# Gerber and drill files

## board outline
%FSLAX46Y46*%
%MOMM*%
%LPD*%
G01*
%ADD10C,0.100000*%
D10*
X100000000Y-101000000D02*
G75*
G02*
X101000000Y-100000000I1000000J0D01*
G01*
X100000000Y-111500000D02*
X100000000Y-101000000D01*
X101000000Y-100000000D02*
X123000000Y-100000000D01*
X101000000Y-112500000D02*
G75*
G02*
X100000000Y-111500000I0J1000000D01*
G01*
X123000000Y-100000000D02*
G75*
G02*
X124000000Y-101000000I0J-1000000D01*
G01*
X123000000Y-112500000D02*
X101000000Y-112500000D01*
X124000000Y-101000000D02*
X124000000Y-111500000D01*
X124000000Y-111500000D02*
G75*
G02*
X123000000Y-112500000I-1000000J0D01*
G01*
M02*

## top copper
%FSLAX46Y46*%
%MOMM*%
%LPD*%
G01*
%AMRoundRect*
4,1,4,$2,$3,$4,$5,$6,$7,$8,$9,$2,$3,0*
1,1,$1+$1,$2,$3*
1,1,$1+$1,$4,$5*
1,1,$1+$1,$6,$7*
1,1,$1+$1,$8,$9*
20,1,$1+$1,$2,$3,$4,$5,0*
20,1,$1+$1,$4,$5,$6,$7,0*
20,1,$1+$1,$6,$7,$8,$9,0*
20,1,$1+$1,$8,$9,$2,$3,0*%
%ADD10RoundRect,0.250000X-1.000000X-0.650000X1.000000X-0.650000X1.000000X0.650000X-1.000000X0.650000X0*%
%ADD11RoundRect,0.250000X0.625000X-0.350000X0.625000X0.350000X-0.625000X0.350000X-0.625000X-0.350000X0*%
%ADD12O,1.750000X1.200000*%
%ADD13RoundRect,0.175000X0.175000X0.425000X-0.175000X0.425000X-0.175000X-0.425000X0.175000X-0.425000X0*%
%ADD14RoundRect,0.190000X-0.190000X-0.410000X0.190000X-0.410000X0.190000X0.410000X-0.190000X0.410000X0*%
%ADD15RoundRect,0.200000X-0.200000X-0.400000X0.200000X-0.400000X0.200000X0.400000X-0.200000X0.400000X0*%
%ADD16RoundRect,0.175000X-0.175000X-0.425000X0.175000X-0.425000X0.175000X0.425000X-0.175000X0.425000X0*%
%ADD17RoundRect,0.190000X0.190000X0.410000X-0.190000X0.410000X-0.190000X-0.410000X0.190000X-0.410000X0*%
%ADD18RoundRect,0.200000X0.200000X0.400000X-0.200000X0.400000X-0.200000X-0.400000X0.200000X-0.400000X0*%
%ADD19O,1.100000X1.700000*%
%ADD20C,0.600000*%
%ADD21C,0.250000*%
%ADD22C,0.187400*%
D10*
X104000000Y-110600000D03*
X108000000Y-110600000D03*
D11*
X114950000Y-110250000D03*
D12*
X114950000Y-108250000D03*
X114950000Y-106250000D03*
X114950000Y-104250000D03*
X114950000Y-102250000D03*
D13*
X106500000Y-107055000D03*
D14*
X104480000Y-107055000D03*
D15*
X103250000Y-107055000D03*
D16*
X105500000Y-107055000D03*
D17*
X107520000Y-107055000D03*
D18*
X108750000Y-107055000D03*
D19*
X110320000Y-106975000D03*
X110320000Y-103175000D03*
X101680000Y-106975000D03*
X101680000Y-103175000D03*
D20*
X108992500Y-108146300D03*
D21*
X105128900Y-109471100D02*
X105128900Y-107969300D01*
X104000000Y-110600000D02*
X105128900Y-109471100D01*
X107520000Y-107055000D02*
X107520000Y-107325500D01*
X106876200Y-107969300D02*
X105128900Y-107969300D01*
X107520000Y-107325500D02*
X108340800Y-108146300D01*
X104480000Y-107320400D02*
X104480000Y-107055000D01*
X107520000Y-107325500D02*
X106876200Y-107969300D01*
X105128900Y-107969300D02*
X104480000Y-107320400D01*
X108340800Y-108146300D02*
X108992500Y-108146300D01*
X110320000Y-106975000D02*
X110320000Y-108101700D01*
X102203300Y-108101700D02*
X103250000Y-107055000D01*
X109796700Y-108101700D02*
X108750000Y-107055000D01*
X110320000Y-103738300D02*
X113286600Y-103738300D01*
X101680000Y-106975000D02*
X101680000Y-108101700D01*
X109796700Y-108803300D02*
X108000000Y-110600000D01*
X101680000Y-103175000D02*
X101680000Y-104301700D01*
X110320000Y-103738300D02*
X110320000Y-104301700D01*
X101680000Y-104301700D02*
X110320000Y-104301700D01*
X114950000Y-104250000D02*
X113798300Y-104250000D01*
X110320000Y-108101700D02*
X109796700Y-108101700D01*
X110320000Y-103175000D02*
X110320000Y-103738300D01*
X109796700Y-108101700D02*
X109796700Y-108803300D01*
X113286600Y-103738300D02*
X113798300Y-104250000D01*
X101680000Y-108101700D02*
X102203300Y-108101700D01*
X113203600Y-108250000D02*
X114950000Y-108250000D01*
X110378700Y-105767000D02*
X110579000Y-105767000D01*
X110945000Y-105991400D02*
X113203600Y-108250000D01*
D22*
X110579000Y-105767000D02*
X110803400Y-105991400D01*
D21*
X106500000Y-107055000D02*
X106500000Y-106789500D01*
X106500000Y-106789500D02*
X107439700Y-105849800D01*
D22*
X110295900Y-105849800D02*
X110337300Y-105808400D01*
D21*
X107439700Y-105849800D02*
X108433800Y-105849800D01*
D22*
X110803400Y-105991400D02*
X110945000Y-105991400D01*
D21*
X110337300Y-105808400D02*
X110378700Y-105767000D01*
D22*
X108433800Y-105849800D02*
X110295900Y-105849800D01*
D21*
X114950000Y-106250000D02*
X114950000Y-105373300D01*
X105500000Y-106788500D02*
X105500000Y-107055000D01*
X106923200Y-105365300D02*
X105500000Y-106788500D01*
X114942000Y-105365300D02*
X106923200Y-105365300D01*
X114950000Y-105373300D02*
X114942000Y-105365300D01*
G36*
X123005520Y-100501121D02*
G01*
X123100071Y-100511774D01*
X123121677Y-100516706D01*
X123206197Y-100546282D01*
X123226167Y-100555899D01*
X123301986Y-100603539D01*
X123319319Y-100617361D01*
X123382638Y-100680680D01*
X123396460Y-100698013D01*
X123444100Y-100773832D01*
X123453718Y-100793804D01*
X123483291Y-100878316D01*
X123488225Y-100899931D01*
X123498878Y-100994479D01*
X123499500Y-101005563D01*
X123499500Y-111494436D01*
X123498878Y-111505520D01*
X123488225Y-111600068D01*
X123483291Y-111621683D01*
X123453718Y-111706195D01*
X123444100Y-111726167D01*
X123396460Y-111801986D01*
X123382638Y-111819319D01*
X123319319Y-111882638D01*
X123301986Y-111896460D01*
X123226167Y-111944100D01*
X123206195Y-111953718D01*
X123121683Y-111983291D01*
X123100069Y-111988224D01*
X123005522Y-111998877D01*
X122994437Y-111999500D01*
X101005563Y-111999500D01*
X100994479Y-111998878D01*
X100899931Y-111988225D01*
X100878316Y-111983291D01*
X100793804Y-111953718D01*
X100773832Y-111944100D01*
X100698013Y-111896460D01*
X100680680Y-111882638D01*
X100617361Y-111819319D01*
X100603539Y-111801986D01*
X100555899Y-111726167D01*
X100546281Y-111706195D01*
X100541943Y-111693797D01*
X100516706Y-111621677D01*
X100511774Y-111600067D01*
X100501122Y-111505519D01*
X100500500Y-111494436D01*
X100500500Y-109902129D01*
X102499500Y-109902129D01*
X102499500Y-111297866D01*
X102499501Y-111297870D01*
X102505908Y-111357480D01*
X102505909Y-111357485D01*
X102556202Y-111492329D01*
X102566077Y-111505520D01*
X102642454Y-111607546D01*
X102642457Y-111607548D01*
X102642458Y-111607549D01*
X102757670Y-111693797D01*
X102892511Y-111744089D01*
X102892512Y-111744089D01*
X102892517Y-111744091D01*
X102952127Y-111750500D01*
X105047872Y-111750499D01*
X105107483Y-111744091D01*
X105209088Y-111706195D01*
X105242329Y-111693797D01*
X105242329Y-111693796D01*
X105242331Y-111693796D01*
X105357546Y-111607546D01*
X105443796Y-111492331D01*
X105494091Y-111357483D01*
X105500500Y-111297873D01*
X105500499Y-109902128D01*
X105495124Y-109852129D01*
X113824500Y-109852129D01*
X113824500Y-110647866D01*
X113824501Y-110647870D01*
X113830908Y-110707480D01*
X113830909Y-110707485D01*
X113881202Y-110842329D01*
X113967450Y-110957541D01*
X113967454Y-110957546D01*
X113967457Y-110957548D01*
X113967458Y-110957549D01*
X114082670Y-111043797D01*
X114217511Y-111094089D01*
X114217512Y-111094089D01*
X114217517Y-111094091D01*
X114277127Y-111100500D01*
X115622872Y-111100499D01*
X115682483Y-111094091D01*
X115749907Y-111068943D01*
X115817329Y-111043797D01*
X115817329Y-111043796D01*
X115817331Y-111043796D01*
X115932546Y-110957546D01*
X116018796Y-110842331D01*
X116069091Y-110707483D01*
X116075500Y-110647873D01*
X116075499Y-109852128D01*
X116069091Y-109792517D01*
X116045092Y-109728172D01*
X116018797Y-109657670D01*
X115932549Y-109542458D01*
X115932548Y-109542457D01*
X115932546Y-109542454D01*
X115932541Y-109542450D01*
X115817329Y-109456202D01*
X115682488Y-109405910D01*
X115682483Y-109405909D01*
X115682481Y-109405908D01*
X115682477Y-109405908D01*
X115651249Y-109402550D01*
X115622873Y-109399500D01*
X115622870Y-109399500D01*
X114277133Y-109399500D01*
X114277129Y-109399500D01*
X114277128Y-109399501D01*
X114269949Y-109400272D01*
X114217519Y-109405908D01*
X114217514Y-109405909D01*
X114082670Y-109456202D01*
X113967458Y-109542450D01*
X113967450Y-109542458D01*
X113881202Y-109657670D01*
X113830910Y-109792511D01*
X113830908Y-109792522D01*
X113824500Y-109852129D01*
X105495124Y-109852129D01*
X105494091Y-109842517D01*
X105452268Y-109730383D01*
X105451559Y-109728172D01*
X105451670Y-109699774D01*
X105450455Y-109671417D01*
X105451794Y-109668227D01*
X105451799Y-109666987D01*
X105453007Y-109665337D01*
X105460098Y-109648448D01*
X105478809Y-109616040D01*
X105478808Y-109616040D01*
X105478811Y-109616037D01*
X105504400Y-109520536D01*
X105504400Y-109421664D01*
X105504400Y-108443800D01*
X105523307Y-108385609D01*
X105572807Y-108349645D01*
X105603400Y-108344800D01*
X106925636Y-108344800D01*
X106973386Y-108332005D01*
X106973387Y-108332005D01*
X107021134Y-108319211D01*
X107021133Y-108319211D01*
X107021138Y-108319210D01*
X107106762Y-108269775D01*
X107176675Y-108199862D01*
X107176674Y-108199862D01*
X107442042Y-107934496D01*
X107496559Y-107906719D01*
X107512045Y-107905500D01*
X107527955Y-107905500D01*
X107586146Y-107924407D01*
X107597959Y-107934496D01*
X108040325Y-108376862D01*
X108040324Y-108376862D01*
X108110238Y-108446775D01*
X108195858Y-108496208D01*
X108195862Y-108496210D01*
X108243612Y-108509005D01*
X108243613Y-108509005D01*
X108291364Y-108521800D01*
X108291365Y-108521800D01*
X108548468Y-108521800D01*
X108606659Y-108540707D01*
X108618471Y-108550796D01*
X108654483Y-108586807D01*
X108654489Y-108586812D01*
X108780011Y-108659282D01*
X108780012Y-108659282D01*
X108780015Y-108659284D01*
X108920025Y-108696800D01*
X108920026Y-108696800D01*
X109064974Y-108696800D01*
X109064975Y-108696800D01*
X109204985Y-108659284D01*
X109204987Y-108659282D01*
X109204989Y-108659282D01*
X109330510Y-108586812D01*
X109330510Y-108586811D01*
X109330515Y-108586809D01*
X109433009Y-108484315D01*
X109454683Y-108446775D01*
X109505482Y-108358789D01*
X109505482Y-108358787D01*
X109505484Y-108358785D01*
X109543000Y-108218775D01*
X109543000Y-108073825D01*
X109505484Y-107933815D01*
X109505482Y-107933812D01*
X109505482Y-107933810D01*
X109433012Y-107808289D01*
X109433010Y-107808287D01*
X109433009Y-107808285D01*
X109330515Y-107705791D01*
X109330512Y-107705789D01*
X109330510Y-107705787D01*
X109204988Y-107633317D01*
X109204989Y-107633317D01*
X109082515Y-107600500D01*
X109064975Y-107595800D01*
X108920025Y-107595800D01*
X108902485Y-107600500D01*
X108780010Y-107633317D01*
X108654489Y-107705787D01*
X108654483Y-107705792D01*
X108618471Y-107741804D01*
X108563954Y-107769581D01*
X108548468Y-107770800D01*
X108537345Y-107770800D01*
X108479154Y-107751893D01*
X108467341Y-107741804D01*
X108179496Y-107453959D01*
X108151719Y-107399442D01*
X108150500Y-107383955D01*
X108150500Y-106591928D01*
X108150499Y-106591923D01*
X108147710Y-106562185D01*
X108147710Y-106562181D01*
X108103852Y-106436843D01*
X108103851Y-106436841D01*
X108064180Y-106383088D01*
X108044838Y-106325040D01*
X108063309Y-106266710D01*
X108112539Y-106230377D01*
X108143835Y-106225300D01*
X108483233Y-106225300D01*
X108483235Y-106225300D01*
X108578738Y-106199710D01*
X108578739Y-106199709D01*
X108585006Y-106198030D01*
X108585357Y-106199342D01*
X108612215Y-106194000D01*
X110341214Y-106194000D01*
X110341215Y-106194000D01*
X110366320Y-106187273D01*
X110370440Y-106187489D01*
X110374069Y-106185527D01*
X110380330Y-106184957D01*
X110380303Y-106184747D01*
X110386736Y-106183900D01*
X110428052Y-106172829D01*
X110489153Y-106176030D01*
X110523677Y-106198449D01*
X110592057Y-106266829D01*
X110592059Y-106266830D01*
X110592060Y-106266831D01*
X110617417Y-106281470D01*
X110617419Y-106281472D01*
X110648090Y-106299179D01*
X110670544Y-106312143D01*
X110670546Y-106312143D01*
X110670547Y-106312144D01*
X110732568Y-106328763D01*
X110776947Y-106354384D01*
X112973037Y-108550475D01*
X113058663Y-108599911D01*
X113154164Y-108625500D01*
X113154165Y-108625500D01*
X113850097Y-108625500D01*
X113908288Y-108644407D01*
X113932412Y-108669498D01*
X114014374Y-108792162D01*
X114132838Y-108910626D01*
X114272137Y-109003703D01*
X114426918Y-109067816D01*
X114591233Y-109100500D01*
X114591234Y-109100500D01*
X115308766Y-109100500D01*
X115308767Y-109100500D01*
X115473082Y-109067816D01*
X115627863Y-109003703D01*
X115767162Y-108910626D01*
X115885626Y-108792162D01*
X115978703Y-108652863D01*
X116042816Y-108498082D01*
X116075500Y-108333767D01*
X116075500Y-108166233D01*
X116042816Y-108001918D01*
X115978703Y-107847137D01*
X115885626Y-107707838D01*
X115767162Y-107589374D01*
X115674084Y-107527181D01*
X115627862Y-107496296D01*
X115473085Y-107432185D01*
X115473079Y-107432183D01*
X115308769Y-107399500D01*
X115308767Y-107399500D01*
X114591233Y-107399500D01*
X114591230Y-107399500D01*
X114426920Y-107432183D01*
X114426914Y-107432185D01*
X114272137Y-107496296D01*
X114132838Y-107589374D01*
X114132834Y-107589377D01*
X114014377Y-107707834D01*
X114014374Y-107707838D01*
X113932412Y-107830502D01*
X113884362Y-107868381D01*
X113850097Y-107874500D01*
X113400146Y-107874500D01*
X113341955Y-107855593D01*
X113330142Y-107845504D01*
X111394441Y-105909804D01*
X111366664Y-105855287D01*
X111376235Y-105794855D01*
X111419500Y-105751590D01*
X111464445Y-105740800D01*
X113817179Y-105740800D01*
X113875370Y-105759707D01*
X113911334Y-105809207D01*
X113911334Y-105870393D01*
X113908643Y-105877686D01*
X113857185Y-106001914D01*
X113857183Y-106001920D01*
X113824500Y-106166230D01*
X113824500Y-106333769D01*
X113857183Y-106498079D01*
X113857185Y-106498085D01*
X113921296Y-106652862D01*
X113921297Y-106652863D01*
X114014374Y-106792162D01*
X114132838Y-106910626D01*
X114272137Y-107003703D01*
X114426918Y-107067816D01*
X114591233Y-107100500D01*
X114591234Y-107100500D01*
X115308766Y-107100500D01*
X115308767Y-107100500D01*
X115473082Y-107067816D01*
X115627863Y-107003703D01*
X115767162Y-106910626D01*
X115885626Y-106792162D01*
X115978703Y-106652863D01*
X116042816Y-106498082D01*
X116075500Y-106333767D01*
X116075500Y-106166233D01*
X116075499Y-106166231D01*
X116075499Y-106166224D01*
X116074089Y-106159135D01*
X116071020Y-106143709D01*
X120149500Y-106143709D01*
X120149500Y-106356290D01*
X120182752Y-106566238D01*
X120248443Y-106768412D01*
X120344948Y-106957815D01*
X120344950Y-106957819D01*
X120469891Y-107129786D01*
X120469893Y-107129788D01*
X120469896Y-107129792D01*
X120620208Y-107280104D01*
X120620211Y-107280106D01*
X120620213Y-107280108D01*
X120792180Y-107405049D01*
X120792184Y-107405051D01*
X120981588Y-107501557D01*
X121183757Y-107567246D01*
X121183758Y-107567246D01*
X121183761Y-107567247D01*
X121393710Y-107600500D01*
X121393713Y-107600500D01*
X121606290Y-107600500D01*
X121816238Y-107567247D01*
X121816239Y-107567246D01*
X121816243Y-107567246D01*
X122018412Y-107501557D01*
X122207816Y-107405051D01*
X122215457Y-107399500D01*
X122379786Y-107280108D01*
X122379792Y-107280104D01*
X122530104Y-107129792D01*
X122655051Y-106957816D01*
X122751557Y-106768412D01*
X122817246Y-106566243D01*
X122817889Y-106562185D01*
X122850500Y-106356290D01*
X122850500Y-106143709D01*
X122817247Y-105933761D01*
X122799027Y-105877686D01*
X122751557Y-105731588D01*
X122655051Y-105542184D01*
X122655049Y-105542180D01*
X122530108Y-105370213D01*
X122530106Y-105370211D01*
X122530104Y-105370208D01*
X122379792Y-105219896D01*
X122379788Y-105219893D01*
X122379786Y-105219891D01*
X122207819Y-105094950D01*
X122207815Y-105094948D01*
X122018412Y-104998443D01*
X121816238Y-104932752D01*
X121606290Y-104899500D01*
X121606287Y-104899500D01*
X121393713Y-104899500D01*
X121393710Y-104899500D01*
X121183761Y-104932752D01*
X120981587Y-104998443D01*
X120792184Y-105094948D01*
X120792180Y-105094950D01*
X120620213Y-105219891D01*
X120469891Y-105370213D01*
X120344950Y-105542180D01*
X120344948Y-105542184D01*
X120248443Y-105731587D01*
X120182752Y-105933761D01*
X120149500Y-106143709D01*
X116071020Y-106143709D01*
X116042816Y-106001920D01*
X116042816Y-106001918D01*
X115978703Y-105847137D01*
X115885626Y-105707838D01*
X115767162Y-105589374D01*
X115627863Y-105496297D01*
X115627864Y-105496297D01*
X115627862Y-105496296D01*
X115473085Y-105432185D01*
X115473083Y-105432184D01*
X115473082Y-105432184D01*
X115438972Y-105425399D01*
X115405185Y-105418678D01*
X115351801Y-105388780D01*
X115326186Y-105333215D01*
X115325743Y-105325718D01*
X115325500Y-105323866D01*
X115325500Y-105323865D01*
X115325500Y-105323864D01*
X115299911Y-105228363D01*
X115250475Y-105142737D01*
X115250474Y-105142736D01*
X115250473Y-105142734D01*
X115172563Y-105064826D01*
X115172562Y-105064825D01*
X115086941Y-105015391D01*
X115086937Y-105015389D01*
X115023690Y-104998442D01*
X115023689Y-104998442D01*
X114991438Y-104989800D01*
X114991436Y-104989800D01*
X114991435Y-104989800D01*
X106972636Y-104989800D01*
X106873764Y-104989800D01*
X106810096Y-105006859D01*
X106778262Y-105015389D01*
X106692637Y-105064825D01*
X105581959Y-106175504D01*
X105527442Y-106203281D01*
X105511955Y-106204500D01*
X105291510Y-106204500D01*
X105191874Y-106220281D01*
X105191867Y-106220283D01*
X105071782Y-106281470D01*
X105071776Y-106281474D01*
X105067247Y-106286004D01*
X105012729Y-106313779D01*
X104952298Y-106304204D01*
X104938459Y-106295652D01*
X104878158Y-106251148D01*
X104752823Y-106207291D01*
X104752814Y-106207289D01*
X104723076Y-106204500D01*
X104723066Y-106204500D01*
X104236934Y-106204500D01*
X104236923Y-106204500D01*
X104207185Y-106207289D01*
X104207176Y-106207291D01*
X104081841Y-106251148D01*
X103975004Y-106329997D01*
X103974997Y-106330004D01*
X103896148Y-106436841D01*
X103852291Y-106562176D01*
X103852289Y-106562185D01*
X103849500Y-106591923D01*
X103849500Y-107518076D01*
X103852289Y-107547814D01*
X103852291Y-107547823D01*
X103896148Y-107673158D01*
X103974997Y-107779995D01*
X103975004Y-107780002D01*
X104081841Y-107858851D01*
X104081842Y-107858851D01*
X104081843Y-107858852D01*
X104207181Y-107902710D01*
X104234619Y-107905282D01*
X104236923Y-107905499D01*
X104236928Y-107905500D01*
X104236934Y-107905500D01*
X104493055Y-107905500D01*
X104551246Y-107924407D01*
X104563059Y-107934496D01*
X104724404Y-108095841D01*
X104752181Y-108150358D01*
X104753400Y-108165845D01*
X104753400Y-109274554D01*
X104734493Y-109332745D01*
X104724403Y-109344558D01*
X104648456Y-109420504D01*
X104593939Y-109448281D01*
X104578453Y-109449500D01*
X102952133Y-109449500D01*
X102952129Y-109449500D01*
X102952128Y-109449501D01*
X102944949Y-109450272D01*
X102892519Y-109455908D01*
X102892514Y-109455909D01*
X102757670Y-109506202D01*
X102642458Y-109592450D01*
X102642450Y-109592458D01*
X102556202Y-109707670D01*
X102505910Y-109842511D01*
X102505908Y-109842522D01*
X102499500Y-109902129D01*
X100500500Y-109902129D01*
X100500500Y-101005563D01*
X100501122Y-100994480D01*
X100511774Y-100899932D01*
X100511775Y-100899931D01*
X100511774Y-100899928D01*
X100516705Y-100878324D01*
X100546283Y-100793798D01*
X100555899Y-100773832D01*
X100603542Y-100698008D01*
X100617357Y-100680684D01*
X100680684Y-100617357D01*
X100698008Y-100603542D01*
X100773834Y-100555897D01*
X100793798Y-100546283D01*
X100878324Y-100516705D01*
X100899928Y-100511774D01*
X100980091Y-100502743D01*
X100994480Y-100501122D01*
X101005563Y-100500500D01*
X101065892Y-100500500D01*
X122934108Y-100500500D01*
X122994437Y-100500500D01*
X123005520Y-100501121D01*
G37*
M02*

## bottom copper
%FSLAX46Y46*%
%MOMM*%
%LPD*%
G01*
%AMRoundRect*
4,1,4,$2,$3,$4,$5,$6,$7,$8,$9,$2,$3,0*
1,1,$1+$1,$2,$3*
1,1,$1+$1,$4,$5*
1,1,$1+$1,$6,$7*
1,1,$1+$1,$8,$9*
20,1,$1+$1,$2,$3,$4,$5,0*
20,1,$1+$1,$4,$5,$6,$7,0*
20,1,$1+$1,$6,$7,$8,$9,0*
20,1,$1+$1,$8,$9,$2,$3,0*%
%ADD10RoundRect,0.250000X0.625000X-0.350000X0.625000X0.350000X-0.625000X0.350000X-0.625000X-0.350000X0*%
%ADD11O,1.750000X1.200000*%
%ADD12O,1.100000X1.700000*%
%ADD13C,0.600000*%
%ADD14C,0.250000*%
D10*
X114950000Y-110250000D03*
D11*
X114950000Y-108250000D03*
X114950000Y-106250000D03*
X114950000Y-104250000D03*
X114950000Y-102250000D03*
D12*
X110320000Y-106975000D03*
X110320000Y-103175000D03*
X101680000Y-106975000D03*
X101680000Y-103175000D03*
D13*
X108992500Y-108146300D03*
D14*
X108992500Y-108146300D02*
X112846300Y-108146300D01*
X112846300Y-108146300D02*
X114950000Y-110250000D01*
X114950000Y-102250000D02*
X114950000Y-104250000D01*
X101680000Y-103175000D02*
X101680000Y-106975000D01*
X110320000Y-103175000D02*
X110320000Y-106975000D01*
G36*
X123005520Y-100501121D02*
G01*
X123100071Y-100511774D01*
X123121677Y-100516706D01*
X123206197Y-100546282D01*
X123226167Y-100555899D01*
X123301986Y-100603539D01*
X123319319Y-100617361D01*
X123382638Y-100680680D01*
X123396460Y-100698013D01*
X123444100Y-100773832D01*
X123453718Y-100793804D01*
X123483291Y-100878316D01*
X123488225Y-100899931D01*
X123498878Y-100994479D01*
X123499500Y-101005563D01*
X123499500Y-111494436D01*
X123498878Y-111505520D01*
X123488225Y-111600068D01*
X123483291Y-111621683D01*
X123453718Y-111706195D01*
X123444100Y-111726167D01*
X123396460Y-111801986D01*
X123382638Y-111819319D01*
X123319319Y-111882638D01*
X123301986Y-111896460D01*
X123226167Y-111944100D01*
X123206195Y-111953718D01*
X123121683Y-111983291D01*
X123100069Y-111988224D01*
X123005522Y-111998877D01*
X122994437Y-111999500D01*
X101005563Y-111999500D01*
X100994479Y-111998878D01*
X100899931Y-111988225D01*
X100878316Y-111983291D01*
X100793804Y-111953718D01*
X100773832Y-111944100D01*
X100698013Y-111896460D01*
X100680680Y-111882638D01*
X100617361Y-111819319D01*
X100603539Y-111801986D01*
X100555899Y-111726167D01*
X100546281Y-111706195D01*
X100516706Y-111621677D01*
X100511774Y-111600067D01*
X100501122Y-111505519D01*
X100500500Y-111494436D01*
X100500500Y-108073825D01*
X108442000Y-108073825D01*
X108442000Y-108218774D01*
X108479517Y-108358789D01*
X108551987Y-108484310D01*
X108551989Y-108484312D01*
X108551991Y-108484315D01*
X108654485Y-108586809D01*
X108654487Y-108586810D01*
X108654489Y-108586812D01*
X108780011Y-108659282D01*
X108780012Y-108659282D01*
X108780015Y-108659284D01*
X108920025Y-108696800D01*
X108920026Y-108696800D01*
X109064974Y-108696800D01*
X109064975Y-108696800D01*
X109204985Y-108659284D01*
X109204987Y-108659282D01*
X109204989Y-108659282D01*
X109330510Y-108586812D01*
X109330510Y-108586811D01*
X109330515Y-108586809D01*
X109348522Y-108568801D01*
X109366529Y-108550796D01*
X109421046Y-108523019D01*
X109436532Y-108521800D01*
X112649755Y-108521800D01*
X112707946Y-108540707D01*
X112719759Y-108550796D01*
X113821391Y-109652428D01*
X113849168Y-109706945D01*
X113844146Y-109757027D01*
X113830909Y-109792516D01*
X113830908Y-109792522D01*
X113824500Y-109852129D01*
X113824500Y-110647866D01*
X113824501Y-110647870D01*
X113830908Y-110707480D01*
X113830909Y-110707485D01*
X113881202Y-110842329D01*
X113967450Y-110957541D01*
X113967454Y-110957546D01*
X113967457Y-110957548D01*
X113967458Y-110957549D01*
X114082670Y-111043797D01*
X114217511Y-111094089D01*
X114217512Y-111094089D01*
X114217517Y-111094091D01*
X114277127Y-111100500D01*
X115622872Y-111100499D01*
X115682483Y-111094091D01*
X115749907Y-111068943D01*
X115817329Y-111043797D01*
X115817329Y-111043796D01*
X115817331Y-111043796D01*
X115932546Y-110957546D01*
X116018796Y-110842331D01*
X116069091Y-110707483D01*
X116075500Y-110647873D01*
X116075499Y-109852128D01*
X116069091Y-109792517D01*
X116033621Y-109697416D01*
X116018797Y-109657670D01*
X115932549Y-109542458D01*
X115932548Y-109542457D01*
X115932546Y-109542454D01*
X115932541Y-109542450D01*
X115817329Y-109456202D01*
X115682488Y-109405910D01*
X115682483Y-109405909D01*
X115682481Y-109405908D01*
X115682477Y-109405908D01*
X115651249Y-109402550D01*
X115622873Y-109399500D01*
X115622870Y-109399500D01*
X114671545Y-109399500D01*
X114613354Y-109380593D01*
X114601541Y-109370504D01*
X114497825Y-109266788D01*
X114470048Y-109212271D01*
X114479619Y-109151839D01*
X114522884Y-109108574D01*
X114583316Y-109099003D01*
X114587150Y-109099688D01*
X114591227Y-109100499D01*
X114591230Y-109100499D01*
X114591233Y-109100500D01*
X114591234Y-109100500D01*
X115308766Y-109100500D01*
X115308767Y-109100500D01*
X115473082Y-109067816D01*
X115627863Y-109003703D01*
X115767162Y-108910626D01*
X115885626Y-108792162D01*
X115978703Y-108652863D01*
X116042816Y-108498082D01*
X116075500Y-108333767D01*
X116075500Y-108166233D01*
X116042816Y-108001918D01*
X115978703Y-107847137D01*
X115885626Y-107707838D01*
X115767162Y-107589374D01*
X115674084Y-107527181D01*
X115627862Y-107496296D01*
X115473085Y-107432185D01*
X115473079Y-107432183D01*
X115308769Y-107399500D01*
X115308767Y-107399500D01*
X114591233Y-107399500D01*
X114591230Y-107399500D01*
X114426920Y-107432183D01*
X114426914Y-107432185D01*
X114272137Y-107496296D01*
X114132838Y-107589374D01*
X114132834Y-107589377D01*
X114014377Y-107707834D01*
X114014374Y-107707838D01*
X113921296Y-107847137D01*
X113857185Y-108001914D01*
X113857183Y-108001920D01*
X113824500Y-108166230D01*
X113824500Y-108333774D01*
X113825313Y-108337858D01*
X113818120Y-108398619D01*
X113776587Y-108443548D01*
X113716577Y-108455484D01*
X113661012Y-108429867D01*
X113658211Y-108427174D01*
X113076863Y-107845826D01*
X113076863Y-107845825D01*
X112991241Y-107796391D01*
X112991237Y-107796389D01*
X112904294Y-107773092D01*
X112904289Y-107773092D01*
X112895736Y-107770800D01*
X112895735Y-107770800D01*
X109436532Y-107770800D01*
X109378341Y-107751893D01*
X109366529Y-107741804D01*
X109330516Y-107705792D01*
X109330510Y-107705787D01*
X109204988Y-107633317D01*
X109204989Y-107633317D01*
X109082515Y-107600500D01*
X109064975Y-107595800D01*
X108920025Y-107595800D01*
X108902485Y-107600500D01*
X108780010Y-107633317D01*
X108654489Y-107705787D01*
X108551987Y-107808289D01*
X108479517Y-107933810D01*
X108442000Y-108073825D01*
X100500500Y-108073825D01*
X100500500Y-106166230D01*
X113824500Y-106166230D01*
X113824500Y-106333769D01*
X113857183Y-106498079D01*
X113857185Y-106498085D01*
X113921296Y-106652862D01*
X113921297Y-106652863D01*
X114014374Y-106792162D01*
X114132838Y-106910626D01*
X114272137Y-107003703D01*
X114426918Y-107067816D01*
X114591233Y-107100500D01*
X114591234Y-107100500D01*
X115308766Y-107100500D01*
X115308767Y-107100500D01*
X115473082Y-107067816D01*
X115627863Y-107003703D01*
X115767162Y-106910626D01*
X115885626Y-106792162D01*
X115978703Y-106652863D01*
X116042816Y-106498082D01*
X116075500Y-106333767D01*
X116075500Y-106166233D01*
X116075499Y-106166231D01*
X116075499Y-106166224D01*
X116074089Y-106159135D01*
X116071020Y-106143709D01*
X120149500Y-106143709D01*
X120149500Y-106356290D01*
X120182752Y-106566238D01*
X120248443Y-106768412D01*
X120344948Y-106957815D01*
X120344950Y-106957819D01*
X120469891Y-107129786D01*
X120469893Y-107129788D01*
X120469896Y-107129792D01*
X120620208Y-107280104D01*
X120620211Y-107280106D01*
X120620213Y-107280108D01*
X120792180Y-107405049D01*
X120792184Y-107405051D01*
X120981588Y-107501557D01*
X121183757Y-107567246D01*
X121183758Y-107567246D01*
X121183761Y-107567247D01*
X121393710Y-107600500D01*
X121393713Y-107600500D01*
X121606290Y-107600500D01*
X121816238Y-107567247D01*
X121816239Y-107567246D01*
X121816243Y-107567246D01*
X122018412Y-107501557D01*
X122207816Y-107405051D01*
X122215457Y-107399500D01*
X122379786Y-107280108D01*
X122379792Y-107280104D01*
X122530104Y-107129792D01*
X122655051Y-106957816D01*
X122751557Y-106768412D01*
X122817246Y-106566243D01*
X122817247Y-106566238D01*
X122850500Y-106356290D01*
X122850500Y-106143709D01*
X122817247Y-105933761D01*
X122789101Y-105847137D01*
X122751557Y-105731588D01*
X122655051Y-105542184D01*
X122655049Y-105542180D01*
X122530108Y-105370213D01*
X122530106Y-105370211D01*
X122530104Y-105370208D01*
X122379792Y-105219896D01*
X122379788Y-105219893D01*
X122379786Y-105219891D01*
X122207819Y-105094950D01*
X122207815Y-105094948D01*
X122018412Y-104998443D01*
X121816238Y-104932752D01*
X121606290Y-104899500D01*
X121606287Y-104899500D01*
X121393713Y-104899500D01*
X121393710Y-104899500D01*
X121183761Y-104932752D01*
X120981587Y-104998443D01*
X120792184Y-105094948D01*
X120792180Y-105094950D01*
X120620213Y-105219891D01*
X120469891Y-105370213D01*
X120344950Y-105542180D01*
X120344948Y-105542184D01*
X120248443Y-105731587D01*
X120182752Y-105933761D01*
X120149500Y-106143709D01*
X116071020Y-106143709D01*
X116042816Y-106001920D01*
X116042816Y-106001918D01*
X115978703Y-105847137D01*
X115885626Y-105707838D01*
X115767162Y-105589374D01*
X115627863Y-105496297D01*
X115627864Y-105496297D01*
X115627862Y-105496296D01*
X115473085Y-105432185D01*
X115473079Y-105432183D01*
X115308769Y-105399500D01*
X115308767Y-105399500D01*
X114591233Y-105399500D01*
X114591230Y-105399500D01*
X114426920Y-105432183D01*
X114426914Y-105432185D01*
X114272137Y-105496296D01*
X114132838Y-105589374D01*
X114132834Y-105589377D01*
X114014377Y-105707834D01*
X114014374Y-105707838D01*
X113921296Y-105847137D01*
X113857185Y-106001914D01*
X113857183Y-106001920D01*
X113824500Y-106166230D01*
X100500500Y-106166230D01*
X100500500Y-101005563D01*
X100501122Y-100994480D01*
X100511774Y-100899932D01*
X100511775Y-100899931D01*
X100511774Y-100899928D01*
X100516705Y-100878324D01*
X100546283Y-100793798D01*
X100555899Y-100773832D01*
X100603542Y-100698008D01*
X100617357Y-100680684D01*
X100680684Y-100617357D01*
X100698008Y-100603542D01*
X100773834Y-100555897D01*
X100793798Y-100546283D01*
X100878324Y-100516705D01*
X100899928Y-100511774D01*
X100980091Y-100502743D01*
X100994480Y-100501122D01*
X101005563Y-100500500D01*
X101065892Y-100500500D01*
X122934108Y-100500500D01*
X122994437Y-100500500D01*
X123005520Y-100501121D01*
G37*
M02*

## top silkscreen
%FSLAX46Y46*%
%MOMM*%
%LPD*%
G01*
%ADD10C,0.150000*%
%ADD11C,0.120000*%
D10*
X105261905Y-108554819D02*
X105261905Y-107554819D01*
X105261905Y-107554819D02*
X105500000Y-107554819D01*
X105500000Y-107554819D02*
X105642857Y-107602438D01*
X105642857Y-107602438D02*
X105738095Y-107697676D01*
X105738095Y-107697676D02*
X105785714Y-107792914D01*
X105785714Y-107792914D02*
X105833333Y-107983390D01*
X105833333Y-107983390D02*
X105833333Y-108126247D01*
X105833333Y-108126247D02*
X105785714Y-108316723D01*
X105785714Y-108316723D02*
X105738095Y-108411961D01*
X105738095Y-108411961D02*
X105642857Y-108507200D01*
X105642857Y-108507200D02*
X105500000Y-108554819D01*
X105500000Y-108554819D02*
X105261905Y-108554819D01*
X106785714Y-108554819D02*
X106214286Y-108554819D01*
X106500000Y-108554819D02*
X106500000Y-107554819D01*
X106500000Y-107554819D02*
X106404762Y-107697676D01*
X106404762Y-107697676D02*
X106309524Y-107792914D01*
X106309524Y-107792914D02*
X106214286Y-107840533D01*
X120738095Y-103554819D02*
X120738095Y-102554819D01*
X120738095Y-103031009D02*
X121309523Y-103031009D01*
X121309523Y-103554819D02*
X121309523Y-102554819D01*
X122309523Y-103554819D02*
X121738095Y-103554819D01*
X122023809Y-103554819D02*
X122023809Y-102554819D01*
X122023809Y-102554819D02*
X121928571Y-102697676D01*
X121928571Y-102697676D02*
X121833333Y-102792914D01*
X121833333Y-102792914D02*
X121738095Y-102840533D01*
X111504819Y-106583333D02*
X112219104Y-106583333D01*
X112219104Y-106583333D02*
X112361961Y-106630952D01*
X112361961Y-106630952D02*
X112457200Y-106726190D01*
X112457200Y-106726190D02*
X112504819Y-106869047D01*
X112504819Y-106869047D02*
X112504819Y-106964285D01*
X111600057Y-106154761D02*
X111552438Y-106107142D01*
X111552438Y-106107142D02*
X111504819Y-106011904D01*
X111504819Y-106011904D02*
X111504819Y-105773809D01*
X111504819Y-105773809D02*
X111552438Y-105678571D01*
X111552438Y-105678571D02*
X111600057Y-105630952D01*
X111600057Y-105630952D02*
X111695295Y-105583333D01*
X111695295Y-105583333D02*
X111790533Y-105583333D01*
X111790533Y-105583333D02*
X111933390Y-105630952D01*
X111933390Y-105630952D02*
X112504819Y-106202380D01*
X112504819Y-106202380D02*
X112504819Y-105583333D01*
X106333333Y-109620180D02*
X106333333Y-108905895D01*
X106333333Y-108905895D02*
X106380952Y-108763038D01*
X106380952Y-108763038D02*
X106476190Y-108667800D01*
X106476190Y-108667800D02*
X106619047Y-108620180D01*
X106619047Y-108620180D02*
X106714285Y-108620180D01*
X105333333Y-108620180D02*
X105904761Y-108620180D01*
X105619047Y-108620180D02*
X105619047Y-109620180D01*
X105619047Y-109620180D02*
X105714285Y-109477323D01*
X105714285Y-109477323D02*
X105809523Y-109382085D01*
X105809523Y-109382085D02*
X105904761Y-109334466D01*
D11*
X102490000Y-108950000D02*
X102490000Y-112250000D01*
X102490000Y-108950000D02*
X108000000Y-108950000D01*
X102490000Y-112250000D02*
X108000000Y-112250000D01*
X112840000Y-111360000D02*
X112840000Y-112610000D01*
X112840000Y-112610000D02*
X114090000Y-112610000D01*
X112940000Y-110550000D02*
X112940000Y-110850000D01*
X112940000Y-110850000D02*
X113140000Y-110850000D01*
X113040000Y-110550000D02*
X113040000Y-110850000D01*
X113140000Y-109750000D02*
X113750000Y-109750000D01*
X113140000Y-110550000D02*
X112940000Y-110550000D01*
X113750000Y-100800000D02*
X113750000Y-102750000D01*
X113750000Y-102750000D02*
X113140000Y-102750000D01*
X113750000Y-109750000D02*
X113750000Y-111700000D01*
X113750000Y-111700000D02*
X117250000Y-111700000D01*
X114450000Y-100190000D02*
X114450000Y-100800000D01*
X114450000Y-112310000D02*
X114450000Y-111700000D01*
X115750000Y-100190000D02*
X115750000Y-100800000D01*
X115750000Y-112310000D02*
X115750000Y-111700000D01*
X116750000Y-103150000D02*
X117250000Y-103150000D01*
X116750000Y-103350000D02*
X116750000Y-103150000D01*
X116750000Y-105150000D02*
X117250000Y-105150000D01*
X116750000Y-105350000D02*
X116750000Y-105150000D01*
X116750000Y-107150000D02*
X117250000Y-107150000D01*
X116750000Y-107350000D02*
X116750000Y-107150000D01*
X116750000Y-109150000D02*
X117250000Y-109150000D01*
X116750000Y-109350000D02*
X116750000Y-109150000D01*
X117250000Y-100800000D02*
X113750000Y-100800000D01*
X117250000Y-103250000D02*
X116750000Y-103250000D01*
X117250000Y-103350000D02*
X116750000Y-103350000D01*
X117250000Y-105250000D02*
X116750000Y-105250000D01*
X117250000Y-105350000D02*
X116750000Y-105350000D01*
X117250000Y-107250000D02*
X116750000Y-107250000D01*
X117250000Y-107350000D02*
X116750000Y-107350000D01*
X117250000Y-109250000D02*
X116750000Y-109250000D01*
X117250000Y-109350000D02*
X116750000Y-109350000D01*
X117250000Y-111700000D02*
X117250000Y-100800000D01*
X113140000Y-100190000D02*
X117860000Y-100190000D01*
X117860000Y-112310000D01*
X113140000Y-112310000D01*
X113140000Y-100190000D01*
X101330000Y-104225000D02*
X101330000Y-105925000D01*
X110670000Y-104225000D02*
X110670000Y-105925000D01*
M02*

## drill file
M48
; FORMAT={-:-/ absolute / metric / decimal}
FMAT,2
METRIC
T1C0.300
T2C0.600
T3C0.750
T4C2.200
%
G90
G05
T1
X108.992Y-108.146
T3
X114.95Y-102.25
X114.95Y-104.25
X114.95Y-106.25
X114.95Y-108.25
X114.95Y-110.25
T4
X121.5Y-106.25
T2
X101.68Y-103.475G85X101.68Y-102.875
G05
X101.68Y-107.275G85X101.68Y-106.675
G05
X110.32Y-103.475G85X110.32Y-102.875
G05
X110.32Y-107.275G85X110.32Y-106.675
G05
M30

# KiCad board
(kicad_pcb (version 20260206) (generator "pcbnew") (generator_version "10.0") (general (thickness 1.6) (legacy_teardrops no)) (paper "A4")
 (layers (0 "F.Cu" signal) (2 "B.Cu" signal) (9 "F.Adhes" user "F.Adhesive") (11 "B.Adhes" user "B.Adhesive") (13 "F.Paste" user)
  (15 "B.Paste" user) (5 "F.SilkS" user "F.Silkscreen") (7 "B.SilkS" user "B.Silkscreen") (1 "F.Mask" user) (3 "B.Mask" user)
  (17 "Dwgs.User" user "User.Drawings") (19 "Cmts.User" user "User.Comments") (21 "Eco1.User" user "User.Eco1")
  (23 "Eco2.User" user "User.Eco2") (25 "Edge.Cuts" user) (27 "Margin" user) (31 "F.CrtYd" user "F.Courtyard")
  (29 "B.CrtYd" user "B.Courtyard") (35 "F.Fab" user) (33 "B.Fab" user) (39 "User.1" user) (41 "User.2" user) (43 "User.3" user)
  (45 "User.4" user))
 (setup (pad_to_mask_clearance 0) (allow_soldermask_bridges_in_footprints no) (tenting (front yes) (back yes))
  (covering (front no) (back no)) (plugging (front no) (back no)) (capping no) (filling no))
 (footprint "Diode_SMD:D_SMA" (layer "F.Cu") (at 106 110.6)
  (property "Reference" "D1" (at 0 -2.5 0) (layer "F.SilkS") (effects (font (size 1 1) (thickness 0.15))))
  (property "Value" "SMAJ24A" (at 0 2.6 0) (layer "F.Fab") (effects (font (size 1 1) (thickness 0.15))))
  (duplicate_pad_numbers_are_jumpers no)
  (fp_line (start -3.51 -1.65) (end -3.51 1.65) (stroke (width 0.12) (type solid)) (layer "F.SilkS"))
  (fp_line (start -3.51 -1.65) (end 2 -1.65) (stroke (width 0.12) (type solid)) (layer "F.SilkS"))
  (fp_line (start -3.51 1.65) (end 2 1.65) (stroke (width 0.12) (type solid)) (layer "F.SilkS"))
  (pad "1" smd roundrect (at -2 0) (size 2.5 1.8) (layers "F.Cu" "F.Mask" "F.Paste") (roundrect_rratio 0.1388888889) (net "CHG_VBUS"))
  (pad "2" smd roundrect (at 2 0) (size 2.5 1.8) (layers "F.Cu" "F.Mask" "F.Paste") (roundrect_rratio 0.1388888889) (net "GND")
   (zone_connect 2)))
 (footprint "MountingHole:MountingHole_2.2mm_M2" (layer "F.Cu") (at 121.5 106.25)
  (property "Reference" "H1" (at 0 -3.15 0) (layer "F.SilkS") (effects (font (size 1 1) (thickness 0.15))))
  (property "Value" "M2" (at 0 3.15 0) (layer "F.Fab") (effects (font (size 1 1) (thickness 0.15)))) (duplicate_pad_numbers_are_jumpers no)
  (pad "" np_thru_hole circle (at 0 0) (size 2.2 2.2) (drill 2.2) (layers "*.Cu" "*.Mask") (zone_connect 2)))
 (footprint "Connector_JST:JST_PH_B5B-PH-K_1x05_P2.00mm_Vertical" (layer "F.Cu") (at 114.95 110.25 90)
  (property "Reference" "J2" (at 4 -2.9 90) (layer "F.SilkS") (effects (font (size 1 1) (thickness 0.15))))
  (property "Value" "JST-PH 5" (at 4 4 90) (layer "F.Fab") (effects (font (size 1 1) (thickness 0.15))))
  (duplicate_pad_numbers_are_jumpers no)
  (fp_line (start -1.11 -2.11) (end -2.36 -2.11) (stroke (width 0.12) (type solid)) (layer "F.SilkS"))
  (fp_line (start -2.36 -2.11) (end -2.36 -0.86) (stroke (width 0.12) (type solid)) (layer "F.SilkS"))
  (fp_line (start -0.3 -2.01) (end -0.6 -2.01) (stroke (width 0.12) (type solid)) (layer "F.SilkS"))
  (fp_line (start -0.6 -2.01) (end -0.6 -1.81) (stroke (width 0.12) (type solid)) (layer "F.SilkS"))
  (fp_line (start -0.3 -1.91) (end -0.6 -1.91) (stroke (width 0.12) (type solid)) (layer "F.SilkS"))
  (fp_line (start 0.5 -1.81) (end 0.5 -1.2) (stroke (width 0.12) (type solid)) (layer "F.SilkS"))
  (fp_line (start -0.3 -1.81) (end -0.3 -2.01) (stroke (width 0.12) (type solid)) (layer "F.SilkS"))
  (fp_line (start 9.45 -1.2) (end 7.5 -1.2) (stroke (width 0.12) (type solid)) (layer "F.SilkS"))
  (fp_line (start 7.5 -1.2) (end 7.5 -1.81) (stroke (width 0.12) (type solid)) (layer "F.SilkS"))
  (fp_line (start 0.5 -1.2) (end -1.45 -1.2) (stroke (width 0.12) (type solid)) (layer "F.SilkS"))
  (fp_line (start -1.45 -1.2) (end -1.45 2.3) (stroke (width 0.12) (type solid)) (layer "F.SilkS"))
  (fp_line (start 10.06 -0.5) (end 9.45 -0.5) (stroke (width 0.12) (type solid)) (layer "F.SilkS"))
  (fp_line (start -2.06 -0.5) (end -1.45 -0.5) (stroke (width 0.12) (type solid)) (layer "F.SilkS"))
  (fp_line (start 10.06 0.8) (end 9.45 0.8) (stroke (width 0.12) (type solid)) (layer "F.SilkS"))
  (fp_line (start -2.06 0.8) (end -1.45 0.8) (stroke (width 0.12) (type solid)) (layer "F.SilkS"))
  (fp_line (start 7.1 1.8) (end 7.1 2.3) (stroke (width 0.12) (type solid)) (layer "F.SilkS"))
  (fp_line (start 6.9 1.8) (end 7.1 1.8) (stroke (width 0.12) (type solid)) (layer "F.SilkS"))
  (fp_line (start 5.1 1.8) (end 5.1 2.3) (stroke (width 0.12) (type solid)) (layer "F.SilkS"))
  (fp_line (start 4.9 1.8) (end 5.1 1.8) (stroke (width 0.12) (type solid)) (layer "F.SilkS"))
  (fp_line (start 3.1 1.8) (end 3.1 2.3) (stroke (width 0.12) (type solid)) (layer "F.SilkS"))
  (fp_line (start 2.9 1.8) (end 3.1 1.8) (stroke (width 0.12) (type solid)) (layer "F.SilkS"))
  (fp_line (start 1.1 1.8) (end 1.1 2.3) (stroke (width 0.12) (type solid)) (layer "F.SilkS"))
  (fp_line (start 0.9 1.8) (end 1.1 1.8) (stroke (width 0.12) (type solid)) (layer "F.SilkS"))
  (fp_line (start 9.45 2.3) (end 9.45 -1.2) (stroke (width 0.12) (type solid)) (layer "F.SilkS"))
  (fp_line (start 7 2.3) (end 7 1.8) (stroke (width 0.12) (type solid)) (layer "F.SilkS"))
  (fp_line (start 6.9 2.3) (end 6.9 1.8) (stroke (width 0.12) (type solid)) (layer "F.SilkS"))
  (fp_line (start 5 2.3) (end 5 1.8) (stroke (width 0.12) (type solid)) (layer "F.SilkS"))
  (fp_line (start 4.9 2.3) (end 4.9 1.8) (stroke (width 0.12) (type solid)) (layer "F.SilkS"))
  (fp_line (start 3 2.3) (end 3 1.8) (stroke (width 0.12) (type solid)) (layer "F.SilkS"))
  (fp_line (start 2.9 2.3) (end 2.9 1.8) (stroke (width 0.12) (type solid)) (layer "F.SilkS"))
  (fp_line (start 1 2.3) (end 1 1.8) (stroke (width 0.12) (type solid)) (layer "F.SilkS"))
  (fp_line (start 0.9 2.3) (end 0.9 1.8) (stroke (width 0.12) (type solid)) (layer "F.SilkS"))
  (fp_line (start -1.45 2.3) (end 9.45 2.3) (stroke (width 0.12) (type solid)) (layer "F.SilkS"))
  (fp_rect (start -2.06 -1.81) (end 10.06 2.91) (stroke (width 0.12) (type solid)) (fill no) (layer "F.SilkS"))
  (pad "1" thru_hole roundrect (at 0 0 90) (size 1.2 1.75) (drill 0.75) (layers "*.Cu" "*.Mask") (remove_unused_layers no)
   (roundrect_rratio 0.208333) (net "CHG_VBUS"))
  (pad "2" thru_hole oval (at 2 0 90) (size 1.2 1.75) (drill 0.75) (layers "*.Cu" "*.Mask") (remove_unused_layers no) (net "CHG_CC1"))
  (pad "3" thru_hole oval (at 4 0 90) (size 1.2 1.75) (drill 0.75) (layers "*.Cu" "*.Mask") (remove_unused_layers no) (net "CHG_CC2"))
  (pad "4" thru_hole oval (at 6 0 90) (size 1.2 1.75) (drill 0.75) (layers "*.Cu" "*.Mask") (remove_unused_layers no) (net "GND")
   (zone_connect 2))
  (pad "5" thru_hole oval (at 8 0 90) (size 1.2 1.75) (drill 0.75) (layers "*.Cu" "*.Mask") (remove_unused_layers no) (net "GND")
   (zone_connect 2)))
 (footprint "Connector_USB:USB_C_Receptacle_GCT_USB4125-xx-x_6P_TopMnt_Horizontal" (layer "F.Cu") (at 106 103.975 180)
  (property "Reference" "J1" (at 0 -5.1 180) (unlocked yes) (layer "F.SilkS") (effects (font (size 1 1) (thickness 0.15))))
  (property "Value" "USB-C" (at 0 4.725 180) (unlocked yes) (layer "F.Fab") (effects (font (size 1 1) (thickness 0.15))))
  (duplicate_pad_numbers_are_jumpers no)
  (fp_line (start 4.67 -0.25) (end 4.67 -1.95) (stroke (width 0.12) (type solid)) (layer "F.SilkS"))
  (fp_line (start -4.67 -0.25) (end -4.67 -1.95) (stroke (width 0.12) (type solid)) (layer "F.SilkS"))
  (pad "A5" smd roundrect (at -0.5 -3.08 180) (size 0.7 1.2) (layers "F.Cu" "F.Mask" "F.Paste") (roundrect_rratio 0.25) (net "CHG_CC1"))
  (pad "A9" smd roundrect (at 1.52 -3.08) (size 0.76 1.2) (layers "F.Cu" "F.Mask" "F.Paste") (roundrect_rratio 0.25) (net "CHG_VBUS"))
  (pad "A12" smd roundrect (at 2.75 -3.08) (size 0.8 1.2) (layers "F.Cu" "F.Mask" "F.Paste") (roundrect_rratio 0.25) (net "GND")
   (zone_connect 2))
  (pad "B5" smd roundrect (at 0.5 -3.08) (size 0.7 1.2) (layers "F.Cu" "F.Mask" "F.Paste") (roundrect_rratio 0.25) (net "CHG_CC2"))
  (pad "B9" smd roundrect (at -1.52 -3.08 180) (size 0.76 1.2) (layers "F.Cu" "F.Mask" "F.Paste") (roundrect_rratio 0.25) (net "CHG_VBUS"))
  (pad "B12" smd roundrect (at -2.75 -3.08 180) (size 0.8 1.2) (layers "F.Cu" "F.Mask" "F.Paste") (roundrect_rratio 0.25) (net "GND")
   (zone_connect 2))
  (pad "SH" thru_hole oval (at -4.32 -3 180) (size 1.1 1.7) (drill oval 0.6 1.2) (layers "*.Cu" "*.Mask" "F.Paste")
   (remove_unused_layers no) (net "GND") (zone_connect 2))
  (pad "SH" thru_hole oval (at -4.32 0.8 180) (size 1.1 1.7) (drill oval 0.6 1.2) (layers "*.Cu" "*.Mask" "F.Paste")
   (remove_unused_layers no) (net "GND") (zone_connect 2))
  (pad "SH" thru_hole oval (at 4.32 -3 180) (size 1.1 1.7) (drill oval 0.6 1.2) (layers "*.Cu" "*.Mask" "F.Paste") (remove_unused_layers no)
   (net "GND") (zone_connect 2))
  (pad "SH" thru_hole oval (at 4.32 0.8 180) (size 1.1 1.7) (drill oval 0.6 1.2) (layers "*.Cu" "*.Mask" "F.Paste")
   (remove_unused_layers no) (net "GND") (zone_connect 2)))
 (gr_arc (start 100 101) (mid 100.292893 100.292893) (end 101 100) (stroke (width 0.1) (type default)) (layer "Edge.Cuts"))
 (gr_line (start 100 111.5) (end 100 101) (stroke (width 0.1) (type default)) (layer "Edge.Cuts"))
 (gr_line (start 101 100) (end 123 100) (stroke (width 0.1) (type default)) (layer "Edge.Cuts"))
 (gr_arc (start 101 112.5) (mid 100.292893 112.207107) (end 100 111.5) (stroke (width 0.1) (type default)) (layer "Edge.Cuts"))
 (gr_arc (start 123 100) (mid 123.707107 100.292893) (end 124 101) (stroke (width 0.1) (type default)) (layer "Edge.Cuts"))
 (gr_line (start 123 112.5) (end 101 112.5) (stroke (width 0.1) (type default)) (layer "Edge.Cuts"))
 (gr_line (start 124 101) (end 124 111.5) (stroke (width 0.1) (type default)) (layer "Edge.Cuts"))
 (gr_arc (start 124 111.5) (mid 123.707107 112.207107) (end 123 112.5) (stroke (width 0.1) (type default)) (layer "Edge.Cuts"))
 (segment (start 105.1289 109.4711) (end 105.1289 107.9693) (width 0.25) (layer "F.Cu") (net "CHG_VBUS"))
 (segment (start 104 110.6) (end 105.1289 109.4711) (width 0.25) (layer "F.Cu") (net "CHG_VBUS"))
 (segment (start 107.52 107.055) (end 107.52 107.3255) (width 0.25) (layer "F.Cu") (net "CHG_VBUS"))
 (segment (start 106.8762 107.9693) (end 105.1289 107.9693) (width 0.25) (layer "F.Cu") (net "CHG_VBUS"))
 (segment (start 107.52 107.3255) (end 108.3408 108.1463) (width 0.25) (layer "F.Cu") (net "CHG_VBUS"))
 (segment (start 104.48 107.3204) (end 104.48 107.055) (width 0.25) (layer "F.Cu") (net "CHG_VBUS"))
 (segment (start 107.52 107.3255) (end 106.8762 107.9693) (width 0.25) (layer "F.Cu") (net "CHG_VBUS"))
 (segment (start 105.1289 107.9693) (end 104.48 107.3204) (width 0.25) (layer "F.Cu") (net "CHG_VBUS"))
 (segment (start 108.3408 108.1463) (end 108.9925 108.1463) (width 0.25) (layer "F.Cu") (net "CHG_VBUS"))
 (via (at 108.9925 108.1463) (size 0.6) (drill 0.3) (layers "F.Cu" "B.Cu") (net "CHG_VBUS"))
 (segment (start 108.9925 108.1463) (end 112.8463 108.1463) (width 0.25) (layer "B.Cu") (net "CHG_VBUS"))
 (segment (start 112.8463 108.1463) (end 114.95 110.25) (width 0.25) (layer "B.Cu") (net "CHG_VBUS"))
 (segment (start 110.32 106.975) (end 110.32 108.1017) (width 0.25) (layer "F.Cu") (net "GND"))
 (segment (start 102.2033 108.1017) (end 103.25 107.055) (width 0.25) (layer "F.Cu") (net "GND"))
 (segment (start 109.7967 108.1017) (end 108.75 107.055) (width 0.25) (layer "F.Cu") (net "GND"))
 (segment (start 110.32 103.7383) (end 113.2866 103.7383) (width 0.25) (layer "F.Cu") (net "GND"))
 (segment (start 101.68 106.975) (end 101.68 108.1017) (width 0.25) (layer "F.Cu") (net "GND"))
 (segment (start 109.7967 108.8033) (end 108 110.6) (width 0.25) (layer "F.Cu") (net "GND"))
 (segment (start 101.68 103.175) (end 101.68 104.3017) (width 0.25) (layer "F.Cu") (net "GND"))
 (segment (start 110.32 103.7383) (end 110.32 104.3017) (width 0.25) (layer "F.Cu") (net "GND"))
 (segment (start 101.68 104.3017) (end 110.32 104.3017) (width 0.25) (layer "F.Cu") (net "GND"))
 (segment (start 114.95 104.25) (end 113.7983 104.25) (width 0.25) (layer "F.Cu") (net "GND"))
 (segment (start 110.32 108.1017) (end 109.7967 108.1017) (width 0.25) (layer "F.Cu") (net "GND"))
 (segment (start 110.32 103.175) (end 110.32 103.7383) (width 0.25) (layer "F.Cu") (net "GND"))
 (segment (start 109.7967 108.1017) (end 109.7967 108.8033) (width 0.25) (layer "F.Cu") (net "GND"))
 (segment (start 113.2866 103.7383) (end 113.7983 104.25) (width 0.25) (layer "F.Cu") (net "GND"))
 (segment (start 101.68 108.1017) (end 102.2033 108.1017) (width 0.25) (layer "F.Cu") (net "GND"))
 (segment (start 114.95 102.25) (end 114.95 104.25) (width 0.25) (layer "B.Cu") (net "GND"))
 (segment (start 101.68 103.175) (end 101.68 106.975) (width 0.25) (layer "B.Cu") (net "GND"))
 (segment (start 110.32 103.175) (end 110.32 106.975) (width 0.25) (layer "B.Cu") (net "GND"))
 (segment (start 113.2036 108.25) (end 114.95 108.25) (width 0.25) (layer "F.Cu") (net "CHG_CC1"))
 (segment (start 110.3787 105.767) (end 110.579 105.767) (width 0.25) (layer "F.Cu") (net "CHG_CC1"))
 (segment (start 110.945 105.9914) (end 113.2036 108.25) (width 0.25) (layer "F.Cu") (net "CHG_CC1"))
 (segment (start 110.579 105.767) (end 110.8034 105.9914) (width 0.1874) (layer "F.Cu") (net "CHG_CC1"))
 (segment (start 106.5 107.055) (end 106.5 106.7895) (width 0.25) (layer "F.Cu") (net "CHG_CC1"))
 (segment (start 106.5 106.7895) (end 107.4397 105.8498) (width 0.25) (layer "F.Cu") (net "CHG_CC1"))
 (segment (start 110.2959 105.8498) (end 110.3373 105.8084) (width 0.1874) (layer "F.Cu") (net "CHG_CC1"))
 (segment (start 107.4397 105.8498) (end 108.4338 105.8498) (width 0.25) (layer "F.Cu") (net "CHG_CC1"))
 (segment (start 110.8034 105.9914) (end 110.945 105.9914) (width 0.1874) (layer "F.Cu") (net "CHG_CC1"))
 (segment (start 110.3373 105.8084) (end 110.3787 105.767) (width 0.25) (layer "F.Cu") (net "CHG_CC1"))
 (segment (start 108.4338 105.8498) (end 110.2959 105.8498) (width 0.1874) (layer "F.Cu") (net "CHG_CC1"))
 (segment (start 114.95 106.25) (end 114.95 105.3733) (width 0.25) (layer "F.Cu") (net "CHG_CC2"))
 (segment (start 105.5 106.7885) (end 105.5 107.055) (width 0.25) (layer "F.Cu") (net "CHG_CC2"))
 (segment (start 106.9232 105.3653) (end 105.5 106.7885) (width 0.25) (layer "F.Cu") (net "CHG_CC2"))
 (segment (start 114.942 105.3653) (end 106.9232 105.3653) (width 0.25) (layer "F.Cu") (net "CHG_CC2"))
 (segment (start 114.95 105.3733) (end 114.942 105.3653) (width 0.25) (layer "F.Cu") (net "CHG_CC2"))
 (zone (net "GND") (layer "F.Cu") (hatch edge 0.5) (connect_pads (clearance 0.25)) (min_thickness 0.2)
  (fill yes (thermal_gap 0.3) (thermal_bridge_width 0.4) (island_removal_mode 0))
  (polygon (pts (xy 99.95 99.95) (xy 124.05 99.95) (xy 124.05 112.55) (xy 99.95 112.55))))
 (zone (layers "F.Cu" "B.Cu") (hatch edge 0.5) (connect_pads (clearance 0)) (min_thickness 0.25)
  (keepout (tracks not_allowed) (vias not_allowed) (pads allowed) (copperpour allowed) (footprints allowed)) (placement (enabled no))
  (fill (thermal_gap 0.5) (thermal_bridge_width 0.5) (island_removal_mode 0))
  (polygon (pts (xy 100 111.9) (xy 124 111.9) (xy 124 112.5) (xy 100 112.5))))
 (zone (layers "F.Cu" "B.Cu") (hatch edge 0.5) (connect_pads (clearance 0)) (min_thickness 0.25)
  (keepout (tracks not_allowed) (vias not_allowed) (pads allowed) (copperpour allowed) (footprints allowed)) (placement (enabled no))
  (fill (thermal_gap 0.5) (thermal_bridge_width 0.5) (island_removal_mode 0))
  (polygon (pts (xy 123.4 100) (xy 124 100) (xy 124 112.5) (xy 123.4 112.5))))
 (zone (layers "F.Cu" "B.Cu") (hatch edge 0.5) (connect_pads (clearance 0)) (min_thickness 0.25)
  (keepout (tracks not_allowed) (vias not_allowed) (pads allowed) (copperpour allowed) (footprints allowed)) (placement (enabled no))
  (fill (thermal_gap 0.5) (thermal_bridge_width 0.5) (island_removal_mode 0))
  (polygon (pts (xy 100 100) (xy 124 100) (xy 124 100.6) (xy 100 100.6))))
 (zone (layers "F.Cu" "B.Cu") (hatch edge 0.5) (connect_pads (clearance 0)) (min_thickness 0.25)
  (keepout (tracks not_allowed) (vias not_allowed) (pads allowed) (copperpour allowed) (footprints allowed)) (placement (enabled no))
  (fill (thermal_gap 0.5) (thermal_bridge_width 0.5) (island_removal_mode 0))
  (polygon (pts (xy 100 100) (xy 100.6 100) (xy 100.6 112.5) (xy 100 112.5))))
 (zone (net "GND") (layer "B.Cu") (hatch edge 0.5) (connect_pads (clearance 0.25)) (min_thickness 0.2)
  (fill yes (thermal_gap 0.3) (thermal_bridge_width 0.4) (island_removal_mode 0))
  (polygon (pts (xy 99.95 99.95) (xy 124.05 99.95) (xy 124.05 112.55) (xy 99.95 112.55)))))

